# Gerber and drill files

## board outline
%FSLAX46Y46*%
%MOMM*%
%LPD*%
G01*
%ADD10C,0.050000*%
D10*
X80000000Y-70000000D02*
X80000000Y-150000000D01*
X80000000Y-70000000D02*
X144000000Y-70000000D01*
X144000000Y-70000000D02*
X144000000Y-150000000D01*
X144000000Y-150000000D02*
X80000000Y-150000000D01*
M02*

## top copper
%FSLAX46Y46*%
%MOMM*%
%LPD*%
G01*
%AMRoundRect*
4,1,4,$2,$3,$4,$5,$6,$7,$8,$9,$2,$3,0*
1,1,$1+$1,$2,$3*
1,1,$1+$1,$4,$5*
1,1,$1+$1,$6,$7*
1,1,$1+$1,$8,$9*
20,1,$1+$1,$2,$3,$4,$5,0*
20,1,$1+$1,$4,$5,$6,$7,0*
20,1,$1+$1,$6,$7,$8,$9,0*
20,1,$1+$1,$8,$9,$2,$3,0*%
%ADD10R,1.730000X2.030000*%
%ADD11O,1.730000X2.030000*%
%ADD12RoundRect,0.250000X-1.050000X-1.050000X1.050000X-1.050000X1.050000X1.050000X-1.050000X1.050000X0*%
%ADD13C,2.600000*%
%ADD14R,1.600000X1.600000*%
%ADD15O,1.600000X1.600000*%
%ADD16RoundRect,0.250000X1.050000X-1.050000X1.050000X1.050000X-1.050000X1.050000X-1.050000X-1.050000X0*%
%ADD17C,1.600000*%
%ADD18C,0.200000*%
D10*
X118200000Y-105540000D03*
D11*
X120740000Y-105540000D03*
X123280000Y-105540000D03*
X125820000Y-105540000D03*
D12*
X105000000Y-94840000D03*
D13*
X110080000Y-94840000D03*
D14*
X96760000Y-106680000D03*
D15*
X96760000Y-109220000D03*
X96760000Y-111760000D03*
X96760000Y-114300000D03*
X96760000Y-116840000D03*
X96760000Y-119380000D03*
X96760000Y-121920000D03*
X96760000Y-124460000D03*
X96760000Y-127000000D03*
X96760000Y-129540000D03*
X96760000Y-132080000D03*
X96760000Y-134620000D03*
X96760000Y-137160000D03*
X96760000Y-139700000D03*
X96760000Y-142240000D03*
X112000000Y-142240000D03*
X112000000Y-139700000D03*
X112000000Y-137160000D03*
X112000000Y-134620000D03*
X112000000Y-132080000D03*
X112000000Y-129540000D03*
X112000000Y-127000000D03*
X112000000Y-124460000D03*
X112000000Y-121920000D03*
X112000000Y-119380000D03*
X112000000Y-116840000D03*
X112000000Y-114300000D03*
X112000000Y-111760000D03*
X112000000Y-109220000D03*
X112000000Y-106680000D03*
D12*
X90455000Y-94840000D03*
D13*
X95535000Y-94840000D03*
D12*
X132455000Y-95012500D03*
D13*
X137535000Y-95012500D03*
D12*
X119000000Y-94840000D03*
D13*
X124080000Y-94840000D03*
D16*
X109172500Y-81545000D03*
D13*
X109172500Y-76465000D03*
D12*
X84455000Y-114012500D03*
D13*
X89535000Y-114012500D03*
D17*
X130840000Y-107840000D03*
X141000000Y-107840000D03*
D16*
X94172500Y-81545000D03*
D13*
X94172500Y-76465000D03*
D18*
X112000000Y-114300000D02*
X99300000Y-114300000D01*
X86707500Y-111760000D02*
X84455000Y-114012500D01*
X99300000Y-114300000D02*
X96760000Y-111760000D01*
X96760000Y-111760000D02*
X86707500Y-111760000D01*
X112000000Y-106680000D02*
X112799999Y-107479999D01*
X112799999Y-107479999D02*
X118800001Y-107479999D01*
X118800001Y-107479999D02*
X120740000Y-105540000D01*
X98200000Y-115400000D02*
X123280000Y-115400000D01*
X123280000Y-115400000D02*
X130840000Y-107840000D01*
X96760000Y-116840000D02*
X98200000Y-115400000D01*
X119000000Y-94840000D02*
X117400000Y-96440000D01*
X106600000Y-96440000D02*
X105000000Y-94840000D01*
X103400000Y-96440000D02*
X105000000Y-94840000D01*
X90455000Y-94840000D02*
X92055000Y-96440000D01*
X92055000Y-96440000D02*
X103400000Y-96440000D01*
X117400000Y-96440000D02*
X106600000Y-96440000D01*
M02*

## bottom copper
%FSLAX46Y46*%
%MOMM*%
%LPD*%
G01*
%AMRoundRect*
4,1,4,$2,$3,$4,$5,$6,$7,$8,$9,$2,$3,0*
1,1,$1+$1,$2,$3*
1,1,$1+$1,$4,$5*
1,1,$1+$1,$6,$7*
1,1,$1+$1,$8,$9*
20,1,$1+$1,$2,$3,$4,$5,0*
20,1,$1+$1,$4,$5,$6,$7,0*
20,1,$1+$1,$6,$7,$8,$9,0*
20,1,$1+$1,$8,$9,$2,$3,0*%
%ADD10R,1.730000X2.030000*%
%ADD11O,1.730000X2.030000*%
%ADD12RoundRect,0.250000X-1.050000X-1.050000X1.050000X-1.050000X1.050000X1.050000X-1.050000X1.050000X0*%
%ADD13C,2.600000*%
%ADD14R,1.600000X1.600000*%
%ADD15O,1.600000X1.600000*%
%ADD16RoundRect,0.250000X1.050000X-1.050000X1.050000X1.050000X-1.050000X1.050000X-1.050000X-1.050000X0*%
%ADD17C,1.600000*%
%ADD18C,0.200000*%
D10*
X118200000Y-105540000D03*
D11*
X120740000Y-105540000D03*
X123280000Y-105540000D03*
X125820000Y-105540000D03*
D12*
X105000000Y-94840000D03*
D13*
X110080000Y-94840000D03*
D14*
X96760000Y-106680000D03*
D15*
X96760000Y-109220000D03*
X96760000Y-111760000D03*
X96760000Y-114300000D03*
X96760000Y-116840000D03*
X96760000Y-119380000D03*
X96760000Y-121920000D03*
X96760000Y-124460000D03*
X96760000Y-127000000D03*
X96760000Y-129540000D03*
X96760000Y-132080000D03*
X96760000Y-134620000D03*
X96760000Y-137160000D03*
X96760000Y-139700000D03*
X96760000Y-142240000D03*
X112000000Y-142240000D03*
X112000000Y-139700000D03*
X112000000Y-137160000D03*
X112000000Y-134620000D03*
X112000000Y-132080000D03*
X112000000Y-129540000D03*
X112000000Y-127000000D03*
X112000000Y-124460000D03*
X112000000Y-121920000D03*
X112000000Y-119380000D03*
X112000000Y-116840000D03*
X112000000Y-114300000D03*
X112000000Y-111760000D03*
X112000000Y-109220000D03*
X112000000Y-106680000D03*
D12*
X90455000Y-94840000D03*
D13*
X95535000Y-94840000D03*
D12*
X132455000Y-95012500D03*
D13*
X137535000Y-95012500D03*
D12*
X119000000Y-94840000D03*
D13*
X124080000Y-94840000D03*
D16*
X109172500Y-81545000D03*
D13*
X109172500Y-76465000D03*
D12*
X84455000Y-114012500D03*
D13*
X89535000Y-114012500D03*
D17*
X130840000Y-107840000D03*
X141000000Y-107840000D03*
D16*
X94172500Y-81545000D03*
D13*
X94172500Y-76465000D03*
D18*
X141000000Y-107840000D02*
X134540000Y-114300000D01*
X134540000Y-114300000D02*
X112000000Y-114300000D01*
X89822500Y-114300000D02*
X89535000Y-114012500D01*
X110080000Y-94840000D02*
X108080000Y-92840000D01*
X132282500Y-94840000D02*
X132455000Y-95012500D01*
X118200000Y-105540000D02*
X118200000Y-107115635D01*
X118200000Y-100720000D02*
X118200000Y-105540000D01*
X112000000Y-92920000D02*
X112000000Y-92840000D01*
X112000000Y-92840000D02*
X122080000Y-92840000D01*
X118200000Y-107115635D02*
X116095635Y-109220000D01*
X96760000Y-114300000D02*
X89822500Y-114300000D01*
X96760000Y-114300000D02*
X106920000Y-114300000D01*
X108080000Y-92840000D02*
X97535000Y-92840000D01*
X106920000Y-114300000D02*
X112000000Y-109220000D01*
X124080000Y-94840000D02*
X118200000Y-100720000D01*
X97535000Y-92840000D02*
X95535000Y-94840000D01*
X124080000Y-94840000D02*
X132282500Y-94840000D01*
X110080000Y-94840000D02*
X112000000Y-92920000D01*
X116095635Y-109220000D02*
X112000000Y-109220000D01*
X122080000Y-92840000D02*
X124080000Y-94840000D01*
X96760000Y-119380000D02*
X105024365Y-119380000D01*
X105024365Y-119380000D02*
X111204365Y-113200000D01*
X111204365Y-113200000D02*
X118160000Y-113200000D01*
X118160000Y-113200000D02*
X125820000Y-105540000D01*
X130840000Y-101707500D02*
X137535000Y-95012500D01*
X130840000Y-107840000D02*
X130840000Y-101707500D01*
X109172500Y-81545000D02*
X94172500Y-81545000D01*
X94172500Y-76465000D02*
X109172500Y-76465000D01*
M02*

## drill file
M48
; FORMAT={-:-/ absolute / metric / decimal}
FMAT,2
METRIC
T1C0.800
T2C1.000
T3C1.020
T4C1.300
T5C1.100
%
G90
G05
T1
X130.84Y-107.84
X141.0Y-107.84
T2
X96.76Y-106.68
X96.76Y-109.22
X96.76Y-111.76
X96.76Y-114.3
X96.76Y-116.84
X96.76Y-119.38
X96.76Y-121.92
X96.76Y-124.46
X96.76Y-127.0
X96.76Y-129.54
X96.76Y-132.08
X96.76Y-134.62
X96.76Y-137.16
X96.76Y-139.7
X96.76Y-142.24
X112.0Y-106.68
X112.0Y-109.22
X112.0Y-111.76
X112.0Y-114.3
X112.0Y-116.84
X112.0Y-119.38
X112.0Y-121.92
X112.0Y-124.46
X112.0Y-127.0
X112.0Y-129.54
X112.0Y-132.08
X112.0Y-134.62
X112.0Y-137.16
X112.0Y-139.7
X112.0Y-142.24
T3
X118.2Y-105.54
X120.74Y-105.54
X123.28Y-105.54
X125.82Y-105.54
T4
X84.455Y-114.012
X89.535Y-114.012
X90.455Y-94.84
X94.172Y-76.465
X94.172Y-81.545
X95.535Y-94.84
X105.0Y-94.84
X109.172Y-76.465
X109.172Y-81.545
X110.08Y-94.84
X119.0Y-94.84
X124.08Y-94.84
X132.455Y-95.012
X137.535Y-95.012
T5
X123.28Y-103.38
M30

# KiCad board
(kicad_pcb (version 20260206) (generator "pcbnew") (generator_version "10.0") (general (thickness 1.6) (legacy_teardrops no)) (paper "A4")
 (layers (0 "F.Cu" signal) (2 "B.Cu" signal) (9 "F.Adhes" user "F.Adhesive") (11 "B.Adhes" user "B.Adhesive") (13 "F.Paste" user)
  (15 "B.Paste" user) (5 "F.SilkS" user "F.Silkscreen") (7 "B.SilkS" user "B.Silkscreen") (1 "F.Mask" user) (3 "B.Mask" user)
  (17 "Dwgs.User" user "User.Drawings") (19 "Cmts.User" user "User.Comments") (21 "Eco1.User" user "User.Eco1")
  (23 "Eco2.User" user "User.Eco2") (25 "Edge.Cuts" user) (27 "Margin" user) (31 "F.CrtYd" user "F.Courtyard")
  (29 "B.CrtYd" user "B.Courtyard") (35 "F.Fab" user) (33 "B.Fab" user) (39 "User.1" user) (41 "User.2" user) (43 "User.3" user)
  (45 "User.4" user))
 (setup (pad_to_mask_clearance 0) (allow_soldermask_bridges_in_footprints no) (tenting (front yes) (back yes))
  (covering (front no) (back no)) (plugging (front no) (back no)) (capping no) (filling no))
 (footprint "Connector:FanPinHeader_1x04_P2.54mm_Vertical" (layer "F.Cu") (at 118.2 105.54)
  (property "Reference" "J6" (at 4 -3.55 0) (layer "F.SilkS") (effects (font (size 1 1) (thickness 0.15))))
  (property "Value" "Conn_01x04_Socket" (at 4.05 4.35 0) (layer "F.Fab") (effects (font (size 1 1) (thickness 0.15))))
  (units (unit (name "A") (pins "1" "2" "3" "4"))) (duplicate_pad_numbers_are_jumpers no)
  (pad "" np_thru_hole circle (at 5.08 -2.16 90) (size 1.1 1.1) (drill 1.1) (layers "*.Cu" "*.Mask"))
  (pad "1" thru_hole rect (at 0 0 90) (size 2.03 1.73) (drill 1.02) (layers "*.Cu" "*.Mask") (remove_unused_layers no) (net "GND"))
  (pad "2" thru_hole oval (at 2.54 0 90) (size 2.03 1.73) (drill 1.02) (layers "*.Cu" "*.Mask") (remove_unused_layers no) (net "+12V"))
  (pad "3" thru_hole oval (at 5.08 0 90) (size 2.03 1.73) (drill 1.02) (layers "*.Cu" "*.Mask") (remove_unused_layers no)
   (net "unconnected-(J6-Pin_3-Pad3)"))
  (pad "4" thru_hole oval (at 7.62 0 90) (size 2.03 1.73) (drill 1.02) (layers "*.Cu" "*.Mask") (remove_unused_layers no) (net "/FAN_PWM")))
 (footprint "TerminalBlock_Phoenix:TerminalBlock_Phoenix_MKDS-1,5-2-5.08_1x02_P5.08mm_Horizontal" (layer "F.Cu") (at 105 94.84)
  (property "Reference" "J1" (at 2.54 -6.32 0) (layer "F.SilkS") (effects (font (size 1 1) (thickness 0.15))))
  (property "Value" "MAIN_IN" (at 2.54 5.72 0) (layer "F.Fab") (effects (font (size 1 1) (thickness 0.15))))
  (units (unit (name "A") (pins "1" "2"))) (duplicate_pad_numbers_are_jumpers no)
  (pad "1" thru_hole roundrect (at 0 0) (size 2.6 2.6) (drill 1.3) (layers "*.Cu" "*.Mask") (remove_unused_layers no)
   (roundrect_rratio 0.096154) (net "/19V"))
  (pad "2" thru_hole circle (at 5.08 0) (size 2.6 2.6) (drill 1.3) (layers "*.Cu" "*.Mask") (remove_unused_layers no) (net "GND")))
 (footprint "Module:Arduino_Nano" (layer "F.Cu") (at 96.76 106.68)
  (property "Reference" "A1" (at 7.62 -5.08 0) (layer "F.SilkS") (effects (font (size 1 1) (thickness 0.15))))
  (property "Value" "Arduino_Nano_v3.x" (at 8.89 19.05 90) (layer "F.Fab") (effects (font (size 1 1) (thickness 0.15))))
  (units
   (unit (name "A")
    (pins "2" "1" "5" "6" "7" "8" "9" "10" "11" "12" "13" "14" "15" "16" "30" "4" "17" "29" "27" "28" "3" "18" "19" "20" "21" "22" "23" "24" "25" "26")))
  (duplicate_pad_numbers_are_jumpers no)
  (pad "1" thru_hole rect (at 0 0) (size 1.6 1.6) (drill 1) (layers "*.Cu" "*.Mask") (remove_unused_layers no)
   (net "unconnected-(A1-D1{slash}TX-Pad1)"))
  (pad "2" thru_hole oval (at 0 2.54) (size 1.6 1.6) (drill 1) (layers "*.Cu" "*.Mask") (remove_unused_layers no)
   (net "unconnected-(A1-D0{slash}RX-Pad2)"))
  (pad "3" thru_hole oval (at 0 5.08) (size 1.6 1.6) (drill 1) (layers "*.Cu" "*.Mask") (remove_unused_layers no) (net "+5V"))
  (pad "4" thru_hole oval (at 0 7.62) (size 1.6 1.6) (drill 1) (layers "*.Cu" "*.Mask") (remove_unused_layers no) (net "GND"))
  (pad "5" thru_hole oval (at 0 10.16) (size 1.6 1.6) (drill 1) (layers "*.Cu" "*.Mask") (remove_unused_layers no) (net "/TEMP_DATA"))
  (pad "6" thru_hole oval (at 0 12.7) (size 1.6 1.6) (drill 1) (layers "*.Cu" "*.Mask") (remove_unused_layers no) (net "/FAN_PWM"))
  (pad "7" thru_hole oval (at 0 15.24) (size 1.6 1.6) (drill 1) (layers "*.Cu" "*.Mask") (remove_unused_layers no)
   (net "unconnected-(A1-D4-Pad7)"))
  (pad "8" thru_hole oval (at 0 17.78) (size 1.6 1.6) (drill 1) (layers "*.Cu" "*.Mask") (remove_unused_layers no)
   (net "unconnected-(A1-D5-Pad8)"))
  (pad "9" thru_hole oval (at 0 20.32) (size 1.6 1.6) (drill 1) (layers "*.Cu" "*.Mask") (remove_unused_layers no)
   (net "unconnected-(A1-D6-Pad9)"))
  (pad "10" thru_hole oval (at 0 22.86) (size 1.6 1.6) (drill 1) (layers "*.Cu" "*.Mask") (remove_unused_layers no)
   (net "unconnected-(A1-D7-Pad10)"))
  (pad "11" thru_hole oval (at 0 25.4) (size 1.6 1.6) (drill 1) (layers "*.Cu" "*.Mask") (remove_unused_layers no)
   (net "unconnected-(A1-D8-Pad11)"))
  (pad "12" thru_hole oval (at 0 27.94) (size 1.6 1.6) (drill 1) (layers "*.Cu" "*.Mask") (remove_unused_layers no)
   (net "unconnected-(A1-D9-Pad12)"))
  (pad "13" thru_hole oval (at 0 30.48) (size 1.6 1.6) (drill 1) (layers "*.Cu" "*.Mask") (remove_unused_layers no)
   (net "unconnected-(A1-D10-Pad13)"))
  (pad "14" thru_hole oval (at 0 33.02) (size 1.6 1.6) (drill 1) (layers "*.Cu" "*.Mask") (remove_unused_layers no)
   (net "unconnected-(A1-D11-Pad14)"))
  (pad "15" thru_hole oval (at 0 35.56) (size 1.6 1.6) (drill 1) (layers "*.Cu" "*.Mask") (remove_unused_layers no)
   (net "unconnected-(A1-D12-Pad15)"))
  (pad "16" thru_hole oval (at 15.24 35.56) (size 1.6 1.6) (drill 1) (layers "*.Cu" "*.Mask") (remove_unused_layers no)
   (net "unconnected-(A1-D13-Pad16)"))
  (pad "17" thru_hole oval (at 15.24 33.02) (size 1.6 1.6) (drill 1) (layers "*.Cu" "*.Mask") (remove_unused_layers no)
   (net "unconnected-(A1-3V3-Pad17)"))
  (pad "18" thru_hole oval (at 15.24 30.48) (size 1.6 1.6) (drill 1) (layers "*.Cu" "*.Mask") (remove_unused_layers no)
   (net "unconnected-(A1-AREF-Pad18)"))
  (pad "19" thru_hole oval (at 15.24 27.94) (size 1.6 1.6) (drill 1) (layers "*.Cu" "*.Mask") (remove_unused_layers no)
   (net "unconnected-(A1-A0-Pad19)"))
  (pad "20" thru_hole oval (at 15.24 25.4) (size 1.6 1.6) (drill 1) (layers "*.Cu" "*.Mask") (remove_unused_layers no)
   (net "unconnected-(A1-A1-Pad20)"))
  (pad "21" thru_hole oval (at 15.24 22.86) (size 1.6 1.6) (drill 1) (layers "*.Cu" "*.Mask") (remove_unused_layers no)
   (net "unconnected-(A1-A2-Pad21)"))
  (pad "22" thru_hole oval (at 15.24 20.32) (size 1.6 1.6) (drill 1) (layers "*.Cu" "*.Mask") (remove_unused_layers no)
   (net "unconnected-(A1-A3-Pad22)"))
  (pad "23" thru_hole oval (at 15.24 17.78) (size 1.6 1.6) (drill 1) (layers "*.Cu" "*.Mask") (remove_unused_layers no)
   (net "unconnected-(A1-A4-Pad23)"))
  (pad "24" thru_hole oval (at 15.24 15.24) (size 1.6 1.6) (drill 1) (layers "*.Cu" "*.Mask") (remove_unused_layers no)
   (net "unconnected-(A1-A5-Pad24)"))
  (pad "25" thru_hole oval (at 15.24 12.7) (size 1.6 1.6) (drill 1) (layers "*.Cu" "*.Mask") (remove_unused_layers no)
   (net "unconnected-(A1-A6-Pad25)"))
  (pad "26" thru_hole oval (at 15.24 10.16) (size 1.6 1.6) (drill 1) (layers "*.Cu" "*.Mask") (remove_unused_layers no)
   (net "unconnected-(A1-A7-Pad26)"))
  (pad "27" thru_hole oval (at 15.24 7.62) (size 1.6 1.6) (drill 1) (layers "*.Cu" "*.Mask") (remove_unused_layers no) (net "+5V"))
  (pad "28" thru_hole oval (at 15.24 5.08) (size 1.6 1.6) (drill 1) (layers "*.Cu" "*.Mask") (remove_unused_layers no)
   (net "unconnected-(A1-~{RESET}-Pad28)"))
  (pad "29" thru_hole oval (at 15.24 2.54) (size 1.6 1.6) (drill 1) (layers "*.Cu" "*.Mask") (remove_unused_layers no) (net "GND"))
  (pad "30" thru_hole oval (at 15.24 0) (size 1.6 1.6) (drill 1) (layers "*.Cu" "*.Mask") (remove_unused_layers no) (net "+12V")))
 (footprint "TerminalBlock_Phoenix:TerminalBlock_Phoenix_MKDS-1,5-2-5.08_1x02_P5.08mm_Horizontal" (layer "F.Cu") (at 90.455 94.84)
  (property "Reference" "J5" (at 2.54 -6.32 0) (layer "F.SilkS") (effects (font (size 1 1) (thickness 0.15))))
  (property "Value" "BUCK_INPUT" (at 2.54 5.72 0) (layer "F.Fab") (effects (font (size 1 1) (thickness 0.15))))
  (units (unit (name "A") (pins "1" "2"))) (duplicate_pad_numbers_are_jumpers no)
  (pad "1" thru_hole roundrect (at 0 0) (size 2.6 2.6) (drill 1.3) (layers "*.Cu" "*.Mask") (remove_unused_layers no)
   (roundrect_rratio 0.096154) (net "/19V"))
  (pad "2" thru_hole circle (at 5.08 0) (size 2.6 2.6) (drill 1.3) (layers "*.Cu" "*.Mask") (remove_unused_layers no) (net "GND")))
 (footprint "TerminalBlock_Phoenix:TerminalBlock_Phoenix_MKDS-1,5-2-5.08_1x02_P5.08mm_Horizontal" (layer "F.Cu") (at 132.455 95.0125)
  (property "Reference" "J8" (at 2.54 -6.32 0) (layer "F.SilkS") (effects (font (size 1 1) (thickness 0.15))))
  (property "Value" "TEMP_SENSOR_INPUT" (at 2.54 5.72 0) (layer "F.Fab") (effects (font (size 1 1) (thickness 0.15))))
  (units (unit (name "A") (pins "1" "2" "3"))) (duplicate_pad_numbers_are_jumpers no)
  (pad "1" thru_hole roundrect (at 0 0) (size 2.6 2.6) (drill 1.3) (layers "*.Cu" "*.Mask") (remove_unused_layers no)
   (roundrect_rratio 0.096154) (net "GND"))
  (pad "2" thru_hole circle (at 5.08 0) (size 2.6 2.6) (drill 1.3) (layers "*.Cu" "*.Mask") (remove_unused_layers no) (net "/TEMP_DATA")))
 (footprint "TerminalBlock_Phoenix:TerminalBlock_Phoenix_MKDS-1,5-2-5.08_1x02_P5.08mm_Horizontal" (layer "F.Cu") (at 119 94.84)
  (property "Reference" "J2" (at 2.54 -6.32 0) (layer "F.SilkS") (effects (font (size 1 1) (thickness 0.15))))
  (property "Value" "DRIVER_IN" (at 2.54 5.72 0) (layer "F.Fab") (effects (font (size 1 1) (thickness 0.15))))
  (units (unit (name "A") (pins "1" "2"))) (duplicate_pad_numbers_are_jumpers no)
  (pad "1" thru_hole roundrect (at 0 0) (size 2.6 2.6) (drill 1.3) (layers "*.Cu" "*.Mask") (remove_unused_layers no)
   (roundrect_rratio 0.096154) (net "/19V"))
  (pad "2" thru_hole circle (at 5.08 0) (size 2.6 2.6) (drill 1.3) (layers "*.Cu" "*.Mask") (remove_unused_layers no) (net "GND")))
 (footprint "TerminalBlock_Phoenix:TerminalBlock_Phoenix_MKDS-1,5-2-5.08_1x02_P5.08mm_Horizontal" (layer "F.Cu") (at 109.1725 81.545 90)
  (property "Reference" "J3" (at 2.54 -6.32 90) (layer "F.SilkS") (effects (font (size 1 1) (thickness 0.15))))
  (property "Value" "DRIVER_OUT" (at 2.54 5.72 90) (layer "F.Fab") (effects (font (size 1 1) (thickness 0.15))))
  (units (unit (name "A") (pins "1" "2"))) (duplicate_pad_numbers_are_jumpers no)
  (pad "1" thru_hole roundrect (at 0 0 90) (size 2.6 2.6) (drill 1.3) (layers "*.Cu" "*.Mask") (remove_unused_layers no)
   (roundrect_rratio 0.096154) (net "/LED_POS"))
  (pad "2" thru_hole circle (at 5.08 0 90) (size 2.6 2.6) (drill 1.3) (layers "*.Cu" "*.Mask") (remove_unused_layers no) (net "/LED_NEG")))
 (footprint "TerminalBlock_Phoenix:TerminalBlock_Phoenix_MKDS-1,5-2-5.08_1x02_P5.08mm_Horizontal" (layer "F.Cu") (at 84.455 114.0125)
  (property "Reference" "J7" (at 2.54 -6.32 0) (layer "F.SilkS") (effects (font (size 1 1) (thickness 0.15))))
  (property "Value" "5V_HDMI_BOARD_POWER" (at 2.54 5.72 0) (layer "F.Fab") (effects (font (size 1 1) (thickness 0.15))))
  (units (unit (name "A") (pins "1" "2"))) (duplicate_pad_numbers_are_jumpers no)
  (pad "1" thru_hole roundrect (at 0 0) (size 2.6 2.6) (drill 1.3) (layers "*.Cu" "*.Mask") (remove_unused_layers no)
   (roundrect_rratio 0.096154) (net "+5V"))
  (pad "2" thru_hole circle (at 5.08 0) (size 2.6 2.6) (drill 1.3) (layers "*.Cu" "*.Mask") (remove_unused_layers no) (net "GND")))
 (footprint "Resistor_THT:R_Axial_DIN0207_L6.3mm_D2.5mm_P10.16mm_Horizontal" (layer "F.Cu") (at 130.84 107.84)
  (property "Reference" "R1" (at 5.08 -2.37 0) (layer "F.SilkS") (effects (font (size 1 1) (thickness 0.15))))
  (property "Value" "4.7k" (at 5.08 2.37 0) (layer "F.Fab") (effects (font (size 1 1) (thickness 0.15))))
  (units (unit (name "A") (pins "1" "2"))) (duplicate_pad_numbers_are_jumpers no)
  (pad "1" thru_hole circle (at 0 0) (size 1.6 1.6) (drill 0.8) (layers "*.Cu" "*.Mask") (remove_unused_layers no) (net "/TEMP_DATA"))
  (pad "2" thru_hole circle (at 10.16 0) (size 1.6 1.6) (drill 0.8) (layers "*.Cu" "*.Mask") (remove_unused_layers no) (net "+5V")))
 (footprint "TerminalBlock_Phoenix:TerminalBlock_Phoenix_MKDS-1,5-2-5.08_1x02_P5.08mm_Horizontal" (layer "F.Cu") (at 94.1725 81.545 90)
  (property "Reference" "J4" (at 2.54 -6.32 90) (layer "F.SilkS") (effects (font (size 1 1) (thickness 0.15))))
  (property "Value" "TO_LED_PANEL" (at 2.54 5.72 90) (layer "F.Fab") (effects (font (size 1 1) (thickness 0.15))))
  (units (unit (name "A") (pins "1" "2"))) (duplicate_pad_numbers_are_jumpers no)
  (pad "1" thru_hole roundrect (at 0 0 90) (size 2.6 2.6) (drill 1.3) (layers "*.Cu" "*.Mask") (remove_unused_layers no)
   (roundrect_rratio 0.096154) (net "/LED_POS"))
  (pad "2" thru_hole circle (at 5.08 0 90) (size 2.6 2.6) (drill 1.3) (layers "*.Cu" "*.Mask") (remove_unused_layers no) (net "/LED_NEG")))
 (gr_line (start 80 70) (end 80 150) (stroke (width 0.05) (type default)) (layer "Edge.Cuts"))
 (gr_line (start 80 70) (end 144 70) (stroke (width 0.05) (type default)) (layer "Edge.Cuts"))
 (gr_line (start 144 70) (end 144 150) (stroke (width 0.05) (type default)) (layer "Edge.Cuts"))
 (gr_line (start 144 150) (end 80 150) (stroke (width 0.05) (type default)) (layer "Edge.Cuts"))
 (segment (start 112 114.3) (end 99.3 114.3) (width 0.2) (layer "F.Cu") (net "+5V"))
 (segment (start 86.7075 111.76) (end 84.455 114.0125) (width 0.2) (layer "F.Cu") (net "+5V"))
 (segment (start 99.3 114.3) (end 96.76 111.76) (width 0.2) (layer "F.Cu") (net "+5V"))
 (segment (start 96.76 111.76) (end 86.7075 111.76) (width 0.2) (layer "F.Cu") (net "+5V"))
 (segment (start 141 107.84) (end 134.54 114.3) (width 0.2) (layer "B.Cu") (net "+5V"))
 (segment (start 134.54 114.3) (end 112 114.3) (width 0.2) (layer "B.Cu") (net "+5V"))
 (segment (start 89.8225 114.3) (end 89.535 114.0125) (width 0.2) (layer "B.Cu") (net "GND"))
 (segment (start 110.08 94.84) (end 108.08 92.84) (width 0.2) (layer "B.Cu") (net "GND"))
 (segment (start 132.2825 94.84) (end 132.455 95.0125) (width 0.2) (layer "B.Cu") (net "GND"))
 (segment (start 118.2 105.54) (end 118.2 107.115635) (width 0.2) (layer "B.Cu") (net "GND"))
 (segment (start 118.2 100.72) (end 118.2 105.54) (width 0.2) (layer "B.Cu") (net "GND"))
 (segment (start 112 92.92) (end 112 92.84) (width 0.2) (layer "B.Cu") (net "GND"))
 (segment (start 112 92.84) (end 122.08 92.84) (width 0.2) (layer "B.Cu") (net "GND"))
 (segment (start 118.2 107.115635) (end 116.095635 109.22) (width 0.2) (layer "B.Cu") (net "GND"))
 (segment (start 96.76 114.3) (end 89.8225 114.3) (width 0.2) (layer "B.Cu") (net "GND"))
 (segment (start 96.76 114.3) (end 106.92 114.3) (width 0.2) (layer "B.Cu") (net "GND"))
 (segment (start 108.08 92.84) (end 97.535 92.84) (width 0.2) (layer "B.Cu") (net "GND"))
 (segment (start 106.92 114.3) (end 112 109.22) (width 0.2) (layer "B.Cu") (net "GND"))
 (segment (start 124.08 94.84) (end 118.2 100.72) (width 0.2) (layer "B.Cu") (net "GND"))
 (segment (start 97.535 92.84) (end 95.535 94.84) (width 0.2) (layer "B.Cu") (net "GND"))
 (segment (start 124.08 94.84) (end 132.2825 94.84) (width 0.2) (layer "B.Cu") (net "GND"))
 (segment (start 110.08 94.84) (end 112 92.92) (width 0.2) (layer "B.Cu") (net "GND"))
 (segment (start 116.095635 109.22) (end 112 109.22) (width 0.2) (layer "B.Cu") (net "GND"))
 (segment (start 122.08 92.84) (end 124.08 94.84) (width 0.2) (layer "B.Cu") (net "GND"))
 (segment (start 112 106.68) (end 112.799999 107.479999) (width 0.2) (layer "F.Cu") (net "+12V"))
 (segment (start 112.799999 107.479999) (end 118.800001 107.479999) (width 0.2) (layer "F.Cu") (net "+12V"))
 (segment (start 118.800001 107.479999) (end 120.74 105.54) (width 0.2) (layer "F.Cu") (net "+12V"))
 (segment (start 96.76 119.38) (end 105.024365 119.38) (width 0.2) (layer "B.Cu") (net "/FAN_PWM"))
 (segment (start 105.024365 119.38) (end 111.204365 113.2) (width 0.2) (layer "B.Cu") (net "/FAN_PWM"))
 (segment (start 111.204365 113.2) (end 118.16 113.2) (width 0.2) (layer "B.Cu") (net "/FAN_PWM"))
 (segment (start 118.16 113.2) (end 125.82 105.54) (width 0.2) (layer "B.Cu") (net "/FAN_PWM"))
 (segment (start 98.2 115.4) (end 123.28 115.4) (width 0.2) (layer "F.Cu") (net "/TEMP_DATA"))
 (segment (start 123.28 115.4) (end 130.84 107.84) (width 0.2) (layer "F.Cu") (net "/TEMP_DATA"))
 (segment (start 96.76 116.84) (end 98.2 115.4) (width 0.2) (layer "F.Cu") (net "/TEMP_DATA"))
 (segment (start 130.84 101.7075) (end 137.535 95.0125) (width 0.2) (layer "B.Cu") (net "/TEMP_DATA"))
 (segment (start 130.84 107.84) (end 130.84 101.7075) (width 0.2) (layer "B.Cu") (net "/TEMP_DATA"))
 (segment (start 119 94.84) (end 117.4 96.44) (width 0.2) (layer "F.Cu") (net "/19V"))
 (segment (start 106.6 96.44) (end 105 94.84) (width 0.2) (layer "F.Cu") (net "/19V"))
 (segment (start 103.4 96.44) (end 105 94.84) (width 0.2) (layer "F.Cu") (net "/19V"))
 (segment (start 90.455 94.84) (end 92.055 96.44) (width 0.2) (layer "F.Cu") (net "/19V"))
 (segment (start 92.055 96.44) (end 103.4 96.44) (width 0.2) (layer "F.Cu") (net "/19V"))
 (segment (start 117.4 96.44) (end 106.6 96.44) (width 0.2) (layer "F.Cu") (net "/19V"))
 (segment (start 109.1725 81.545) (end 94.1725 81.545) (width 0.2) (layer "B.Cu") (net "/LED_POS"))
 (segment (start 94.1725 76.465) (end 109.1725 76.465) (width 0.2) (layer "B.Cu") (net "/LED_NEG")))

